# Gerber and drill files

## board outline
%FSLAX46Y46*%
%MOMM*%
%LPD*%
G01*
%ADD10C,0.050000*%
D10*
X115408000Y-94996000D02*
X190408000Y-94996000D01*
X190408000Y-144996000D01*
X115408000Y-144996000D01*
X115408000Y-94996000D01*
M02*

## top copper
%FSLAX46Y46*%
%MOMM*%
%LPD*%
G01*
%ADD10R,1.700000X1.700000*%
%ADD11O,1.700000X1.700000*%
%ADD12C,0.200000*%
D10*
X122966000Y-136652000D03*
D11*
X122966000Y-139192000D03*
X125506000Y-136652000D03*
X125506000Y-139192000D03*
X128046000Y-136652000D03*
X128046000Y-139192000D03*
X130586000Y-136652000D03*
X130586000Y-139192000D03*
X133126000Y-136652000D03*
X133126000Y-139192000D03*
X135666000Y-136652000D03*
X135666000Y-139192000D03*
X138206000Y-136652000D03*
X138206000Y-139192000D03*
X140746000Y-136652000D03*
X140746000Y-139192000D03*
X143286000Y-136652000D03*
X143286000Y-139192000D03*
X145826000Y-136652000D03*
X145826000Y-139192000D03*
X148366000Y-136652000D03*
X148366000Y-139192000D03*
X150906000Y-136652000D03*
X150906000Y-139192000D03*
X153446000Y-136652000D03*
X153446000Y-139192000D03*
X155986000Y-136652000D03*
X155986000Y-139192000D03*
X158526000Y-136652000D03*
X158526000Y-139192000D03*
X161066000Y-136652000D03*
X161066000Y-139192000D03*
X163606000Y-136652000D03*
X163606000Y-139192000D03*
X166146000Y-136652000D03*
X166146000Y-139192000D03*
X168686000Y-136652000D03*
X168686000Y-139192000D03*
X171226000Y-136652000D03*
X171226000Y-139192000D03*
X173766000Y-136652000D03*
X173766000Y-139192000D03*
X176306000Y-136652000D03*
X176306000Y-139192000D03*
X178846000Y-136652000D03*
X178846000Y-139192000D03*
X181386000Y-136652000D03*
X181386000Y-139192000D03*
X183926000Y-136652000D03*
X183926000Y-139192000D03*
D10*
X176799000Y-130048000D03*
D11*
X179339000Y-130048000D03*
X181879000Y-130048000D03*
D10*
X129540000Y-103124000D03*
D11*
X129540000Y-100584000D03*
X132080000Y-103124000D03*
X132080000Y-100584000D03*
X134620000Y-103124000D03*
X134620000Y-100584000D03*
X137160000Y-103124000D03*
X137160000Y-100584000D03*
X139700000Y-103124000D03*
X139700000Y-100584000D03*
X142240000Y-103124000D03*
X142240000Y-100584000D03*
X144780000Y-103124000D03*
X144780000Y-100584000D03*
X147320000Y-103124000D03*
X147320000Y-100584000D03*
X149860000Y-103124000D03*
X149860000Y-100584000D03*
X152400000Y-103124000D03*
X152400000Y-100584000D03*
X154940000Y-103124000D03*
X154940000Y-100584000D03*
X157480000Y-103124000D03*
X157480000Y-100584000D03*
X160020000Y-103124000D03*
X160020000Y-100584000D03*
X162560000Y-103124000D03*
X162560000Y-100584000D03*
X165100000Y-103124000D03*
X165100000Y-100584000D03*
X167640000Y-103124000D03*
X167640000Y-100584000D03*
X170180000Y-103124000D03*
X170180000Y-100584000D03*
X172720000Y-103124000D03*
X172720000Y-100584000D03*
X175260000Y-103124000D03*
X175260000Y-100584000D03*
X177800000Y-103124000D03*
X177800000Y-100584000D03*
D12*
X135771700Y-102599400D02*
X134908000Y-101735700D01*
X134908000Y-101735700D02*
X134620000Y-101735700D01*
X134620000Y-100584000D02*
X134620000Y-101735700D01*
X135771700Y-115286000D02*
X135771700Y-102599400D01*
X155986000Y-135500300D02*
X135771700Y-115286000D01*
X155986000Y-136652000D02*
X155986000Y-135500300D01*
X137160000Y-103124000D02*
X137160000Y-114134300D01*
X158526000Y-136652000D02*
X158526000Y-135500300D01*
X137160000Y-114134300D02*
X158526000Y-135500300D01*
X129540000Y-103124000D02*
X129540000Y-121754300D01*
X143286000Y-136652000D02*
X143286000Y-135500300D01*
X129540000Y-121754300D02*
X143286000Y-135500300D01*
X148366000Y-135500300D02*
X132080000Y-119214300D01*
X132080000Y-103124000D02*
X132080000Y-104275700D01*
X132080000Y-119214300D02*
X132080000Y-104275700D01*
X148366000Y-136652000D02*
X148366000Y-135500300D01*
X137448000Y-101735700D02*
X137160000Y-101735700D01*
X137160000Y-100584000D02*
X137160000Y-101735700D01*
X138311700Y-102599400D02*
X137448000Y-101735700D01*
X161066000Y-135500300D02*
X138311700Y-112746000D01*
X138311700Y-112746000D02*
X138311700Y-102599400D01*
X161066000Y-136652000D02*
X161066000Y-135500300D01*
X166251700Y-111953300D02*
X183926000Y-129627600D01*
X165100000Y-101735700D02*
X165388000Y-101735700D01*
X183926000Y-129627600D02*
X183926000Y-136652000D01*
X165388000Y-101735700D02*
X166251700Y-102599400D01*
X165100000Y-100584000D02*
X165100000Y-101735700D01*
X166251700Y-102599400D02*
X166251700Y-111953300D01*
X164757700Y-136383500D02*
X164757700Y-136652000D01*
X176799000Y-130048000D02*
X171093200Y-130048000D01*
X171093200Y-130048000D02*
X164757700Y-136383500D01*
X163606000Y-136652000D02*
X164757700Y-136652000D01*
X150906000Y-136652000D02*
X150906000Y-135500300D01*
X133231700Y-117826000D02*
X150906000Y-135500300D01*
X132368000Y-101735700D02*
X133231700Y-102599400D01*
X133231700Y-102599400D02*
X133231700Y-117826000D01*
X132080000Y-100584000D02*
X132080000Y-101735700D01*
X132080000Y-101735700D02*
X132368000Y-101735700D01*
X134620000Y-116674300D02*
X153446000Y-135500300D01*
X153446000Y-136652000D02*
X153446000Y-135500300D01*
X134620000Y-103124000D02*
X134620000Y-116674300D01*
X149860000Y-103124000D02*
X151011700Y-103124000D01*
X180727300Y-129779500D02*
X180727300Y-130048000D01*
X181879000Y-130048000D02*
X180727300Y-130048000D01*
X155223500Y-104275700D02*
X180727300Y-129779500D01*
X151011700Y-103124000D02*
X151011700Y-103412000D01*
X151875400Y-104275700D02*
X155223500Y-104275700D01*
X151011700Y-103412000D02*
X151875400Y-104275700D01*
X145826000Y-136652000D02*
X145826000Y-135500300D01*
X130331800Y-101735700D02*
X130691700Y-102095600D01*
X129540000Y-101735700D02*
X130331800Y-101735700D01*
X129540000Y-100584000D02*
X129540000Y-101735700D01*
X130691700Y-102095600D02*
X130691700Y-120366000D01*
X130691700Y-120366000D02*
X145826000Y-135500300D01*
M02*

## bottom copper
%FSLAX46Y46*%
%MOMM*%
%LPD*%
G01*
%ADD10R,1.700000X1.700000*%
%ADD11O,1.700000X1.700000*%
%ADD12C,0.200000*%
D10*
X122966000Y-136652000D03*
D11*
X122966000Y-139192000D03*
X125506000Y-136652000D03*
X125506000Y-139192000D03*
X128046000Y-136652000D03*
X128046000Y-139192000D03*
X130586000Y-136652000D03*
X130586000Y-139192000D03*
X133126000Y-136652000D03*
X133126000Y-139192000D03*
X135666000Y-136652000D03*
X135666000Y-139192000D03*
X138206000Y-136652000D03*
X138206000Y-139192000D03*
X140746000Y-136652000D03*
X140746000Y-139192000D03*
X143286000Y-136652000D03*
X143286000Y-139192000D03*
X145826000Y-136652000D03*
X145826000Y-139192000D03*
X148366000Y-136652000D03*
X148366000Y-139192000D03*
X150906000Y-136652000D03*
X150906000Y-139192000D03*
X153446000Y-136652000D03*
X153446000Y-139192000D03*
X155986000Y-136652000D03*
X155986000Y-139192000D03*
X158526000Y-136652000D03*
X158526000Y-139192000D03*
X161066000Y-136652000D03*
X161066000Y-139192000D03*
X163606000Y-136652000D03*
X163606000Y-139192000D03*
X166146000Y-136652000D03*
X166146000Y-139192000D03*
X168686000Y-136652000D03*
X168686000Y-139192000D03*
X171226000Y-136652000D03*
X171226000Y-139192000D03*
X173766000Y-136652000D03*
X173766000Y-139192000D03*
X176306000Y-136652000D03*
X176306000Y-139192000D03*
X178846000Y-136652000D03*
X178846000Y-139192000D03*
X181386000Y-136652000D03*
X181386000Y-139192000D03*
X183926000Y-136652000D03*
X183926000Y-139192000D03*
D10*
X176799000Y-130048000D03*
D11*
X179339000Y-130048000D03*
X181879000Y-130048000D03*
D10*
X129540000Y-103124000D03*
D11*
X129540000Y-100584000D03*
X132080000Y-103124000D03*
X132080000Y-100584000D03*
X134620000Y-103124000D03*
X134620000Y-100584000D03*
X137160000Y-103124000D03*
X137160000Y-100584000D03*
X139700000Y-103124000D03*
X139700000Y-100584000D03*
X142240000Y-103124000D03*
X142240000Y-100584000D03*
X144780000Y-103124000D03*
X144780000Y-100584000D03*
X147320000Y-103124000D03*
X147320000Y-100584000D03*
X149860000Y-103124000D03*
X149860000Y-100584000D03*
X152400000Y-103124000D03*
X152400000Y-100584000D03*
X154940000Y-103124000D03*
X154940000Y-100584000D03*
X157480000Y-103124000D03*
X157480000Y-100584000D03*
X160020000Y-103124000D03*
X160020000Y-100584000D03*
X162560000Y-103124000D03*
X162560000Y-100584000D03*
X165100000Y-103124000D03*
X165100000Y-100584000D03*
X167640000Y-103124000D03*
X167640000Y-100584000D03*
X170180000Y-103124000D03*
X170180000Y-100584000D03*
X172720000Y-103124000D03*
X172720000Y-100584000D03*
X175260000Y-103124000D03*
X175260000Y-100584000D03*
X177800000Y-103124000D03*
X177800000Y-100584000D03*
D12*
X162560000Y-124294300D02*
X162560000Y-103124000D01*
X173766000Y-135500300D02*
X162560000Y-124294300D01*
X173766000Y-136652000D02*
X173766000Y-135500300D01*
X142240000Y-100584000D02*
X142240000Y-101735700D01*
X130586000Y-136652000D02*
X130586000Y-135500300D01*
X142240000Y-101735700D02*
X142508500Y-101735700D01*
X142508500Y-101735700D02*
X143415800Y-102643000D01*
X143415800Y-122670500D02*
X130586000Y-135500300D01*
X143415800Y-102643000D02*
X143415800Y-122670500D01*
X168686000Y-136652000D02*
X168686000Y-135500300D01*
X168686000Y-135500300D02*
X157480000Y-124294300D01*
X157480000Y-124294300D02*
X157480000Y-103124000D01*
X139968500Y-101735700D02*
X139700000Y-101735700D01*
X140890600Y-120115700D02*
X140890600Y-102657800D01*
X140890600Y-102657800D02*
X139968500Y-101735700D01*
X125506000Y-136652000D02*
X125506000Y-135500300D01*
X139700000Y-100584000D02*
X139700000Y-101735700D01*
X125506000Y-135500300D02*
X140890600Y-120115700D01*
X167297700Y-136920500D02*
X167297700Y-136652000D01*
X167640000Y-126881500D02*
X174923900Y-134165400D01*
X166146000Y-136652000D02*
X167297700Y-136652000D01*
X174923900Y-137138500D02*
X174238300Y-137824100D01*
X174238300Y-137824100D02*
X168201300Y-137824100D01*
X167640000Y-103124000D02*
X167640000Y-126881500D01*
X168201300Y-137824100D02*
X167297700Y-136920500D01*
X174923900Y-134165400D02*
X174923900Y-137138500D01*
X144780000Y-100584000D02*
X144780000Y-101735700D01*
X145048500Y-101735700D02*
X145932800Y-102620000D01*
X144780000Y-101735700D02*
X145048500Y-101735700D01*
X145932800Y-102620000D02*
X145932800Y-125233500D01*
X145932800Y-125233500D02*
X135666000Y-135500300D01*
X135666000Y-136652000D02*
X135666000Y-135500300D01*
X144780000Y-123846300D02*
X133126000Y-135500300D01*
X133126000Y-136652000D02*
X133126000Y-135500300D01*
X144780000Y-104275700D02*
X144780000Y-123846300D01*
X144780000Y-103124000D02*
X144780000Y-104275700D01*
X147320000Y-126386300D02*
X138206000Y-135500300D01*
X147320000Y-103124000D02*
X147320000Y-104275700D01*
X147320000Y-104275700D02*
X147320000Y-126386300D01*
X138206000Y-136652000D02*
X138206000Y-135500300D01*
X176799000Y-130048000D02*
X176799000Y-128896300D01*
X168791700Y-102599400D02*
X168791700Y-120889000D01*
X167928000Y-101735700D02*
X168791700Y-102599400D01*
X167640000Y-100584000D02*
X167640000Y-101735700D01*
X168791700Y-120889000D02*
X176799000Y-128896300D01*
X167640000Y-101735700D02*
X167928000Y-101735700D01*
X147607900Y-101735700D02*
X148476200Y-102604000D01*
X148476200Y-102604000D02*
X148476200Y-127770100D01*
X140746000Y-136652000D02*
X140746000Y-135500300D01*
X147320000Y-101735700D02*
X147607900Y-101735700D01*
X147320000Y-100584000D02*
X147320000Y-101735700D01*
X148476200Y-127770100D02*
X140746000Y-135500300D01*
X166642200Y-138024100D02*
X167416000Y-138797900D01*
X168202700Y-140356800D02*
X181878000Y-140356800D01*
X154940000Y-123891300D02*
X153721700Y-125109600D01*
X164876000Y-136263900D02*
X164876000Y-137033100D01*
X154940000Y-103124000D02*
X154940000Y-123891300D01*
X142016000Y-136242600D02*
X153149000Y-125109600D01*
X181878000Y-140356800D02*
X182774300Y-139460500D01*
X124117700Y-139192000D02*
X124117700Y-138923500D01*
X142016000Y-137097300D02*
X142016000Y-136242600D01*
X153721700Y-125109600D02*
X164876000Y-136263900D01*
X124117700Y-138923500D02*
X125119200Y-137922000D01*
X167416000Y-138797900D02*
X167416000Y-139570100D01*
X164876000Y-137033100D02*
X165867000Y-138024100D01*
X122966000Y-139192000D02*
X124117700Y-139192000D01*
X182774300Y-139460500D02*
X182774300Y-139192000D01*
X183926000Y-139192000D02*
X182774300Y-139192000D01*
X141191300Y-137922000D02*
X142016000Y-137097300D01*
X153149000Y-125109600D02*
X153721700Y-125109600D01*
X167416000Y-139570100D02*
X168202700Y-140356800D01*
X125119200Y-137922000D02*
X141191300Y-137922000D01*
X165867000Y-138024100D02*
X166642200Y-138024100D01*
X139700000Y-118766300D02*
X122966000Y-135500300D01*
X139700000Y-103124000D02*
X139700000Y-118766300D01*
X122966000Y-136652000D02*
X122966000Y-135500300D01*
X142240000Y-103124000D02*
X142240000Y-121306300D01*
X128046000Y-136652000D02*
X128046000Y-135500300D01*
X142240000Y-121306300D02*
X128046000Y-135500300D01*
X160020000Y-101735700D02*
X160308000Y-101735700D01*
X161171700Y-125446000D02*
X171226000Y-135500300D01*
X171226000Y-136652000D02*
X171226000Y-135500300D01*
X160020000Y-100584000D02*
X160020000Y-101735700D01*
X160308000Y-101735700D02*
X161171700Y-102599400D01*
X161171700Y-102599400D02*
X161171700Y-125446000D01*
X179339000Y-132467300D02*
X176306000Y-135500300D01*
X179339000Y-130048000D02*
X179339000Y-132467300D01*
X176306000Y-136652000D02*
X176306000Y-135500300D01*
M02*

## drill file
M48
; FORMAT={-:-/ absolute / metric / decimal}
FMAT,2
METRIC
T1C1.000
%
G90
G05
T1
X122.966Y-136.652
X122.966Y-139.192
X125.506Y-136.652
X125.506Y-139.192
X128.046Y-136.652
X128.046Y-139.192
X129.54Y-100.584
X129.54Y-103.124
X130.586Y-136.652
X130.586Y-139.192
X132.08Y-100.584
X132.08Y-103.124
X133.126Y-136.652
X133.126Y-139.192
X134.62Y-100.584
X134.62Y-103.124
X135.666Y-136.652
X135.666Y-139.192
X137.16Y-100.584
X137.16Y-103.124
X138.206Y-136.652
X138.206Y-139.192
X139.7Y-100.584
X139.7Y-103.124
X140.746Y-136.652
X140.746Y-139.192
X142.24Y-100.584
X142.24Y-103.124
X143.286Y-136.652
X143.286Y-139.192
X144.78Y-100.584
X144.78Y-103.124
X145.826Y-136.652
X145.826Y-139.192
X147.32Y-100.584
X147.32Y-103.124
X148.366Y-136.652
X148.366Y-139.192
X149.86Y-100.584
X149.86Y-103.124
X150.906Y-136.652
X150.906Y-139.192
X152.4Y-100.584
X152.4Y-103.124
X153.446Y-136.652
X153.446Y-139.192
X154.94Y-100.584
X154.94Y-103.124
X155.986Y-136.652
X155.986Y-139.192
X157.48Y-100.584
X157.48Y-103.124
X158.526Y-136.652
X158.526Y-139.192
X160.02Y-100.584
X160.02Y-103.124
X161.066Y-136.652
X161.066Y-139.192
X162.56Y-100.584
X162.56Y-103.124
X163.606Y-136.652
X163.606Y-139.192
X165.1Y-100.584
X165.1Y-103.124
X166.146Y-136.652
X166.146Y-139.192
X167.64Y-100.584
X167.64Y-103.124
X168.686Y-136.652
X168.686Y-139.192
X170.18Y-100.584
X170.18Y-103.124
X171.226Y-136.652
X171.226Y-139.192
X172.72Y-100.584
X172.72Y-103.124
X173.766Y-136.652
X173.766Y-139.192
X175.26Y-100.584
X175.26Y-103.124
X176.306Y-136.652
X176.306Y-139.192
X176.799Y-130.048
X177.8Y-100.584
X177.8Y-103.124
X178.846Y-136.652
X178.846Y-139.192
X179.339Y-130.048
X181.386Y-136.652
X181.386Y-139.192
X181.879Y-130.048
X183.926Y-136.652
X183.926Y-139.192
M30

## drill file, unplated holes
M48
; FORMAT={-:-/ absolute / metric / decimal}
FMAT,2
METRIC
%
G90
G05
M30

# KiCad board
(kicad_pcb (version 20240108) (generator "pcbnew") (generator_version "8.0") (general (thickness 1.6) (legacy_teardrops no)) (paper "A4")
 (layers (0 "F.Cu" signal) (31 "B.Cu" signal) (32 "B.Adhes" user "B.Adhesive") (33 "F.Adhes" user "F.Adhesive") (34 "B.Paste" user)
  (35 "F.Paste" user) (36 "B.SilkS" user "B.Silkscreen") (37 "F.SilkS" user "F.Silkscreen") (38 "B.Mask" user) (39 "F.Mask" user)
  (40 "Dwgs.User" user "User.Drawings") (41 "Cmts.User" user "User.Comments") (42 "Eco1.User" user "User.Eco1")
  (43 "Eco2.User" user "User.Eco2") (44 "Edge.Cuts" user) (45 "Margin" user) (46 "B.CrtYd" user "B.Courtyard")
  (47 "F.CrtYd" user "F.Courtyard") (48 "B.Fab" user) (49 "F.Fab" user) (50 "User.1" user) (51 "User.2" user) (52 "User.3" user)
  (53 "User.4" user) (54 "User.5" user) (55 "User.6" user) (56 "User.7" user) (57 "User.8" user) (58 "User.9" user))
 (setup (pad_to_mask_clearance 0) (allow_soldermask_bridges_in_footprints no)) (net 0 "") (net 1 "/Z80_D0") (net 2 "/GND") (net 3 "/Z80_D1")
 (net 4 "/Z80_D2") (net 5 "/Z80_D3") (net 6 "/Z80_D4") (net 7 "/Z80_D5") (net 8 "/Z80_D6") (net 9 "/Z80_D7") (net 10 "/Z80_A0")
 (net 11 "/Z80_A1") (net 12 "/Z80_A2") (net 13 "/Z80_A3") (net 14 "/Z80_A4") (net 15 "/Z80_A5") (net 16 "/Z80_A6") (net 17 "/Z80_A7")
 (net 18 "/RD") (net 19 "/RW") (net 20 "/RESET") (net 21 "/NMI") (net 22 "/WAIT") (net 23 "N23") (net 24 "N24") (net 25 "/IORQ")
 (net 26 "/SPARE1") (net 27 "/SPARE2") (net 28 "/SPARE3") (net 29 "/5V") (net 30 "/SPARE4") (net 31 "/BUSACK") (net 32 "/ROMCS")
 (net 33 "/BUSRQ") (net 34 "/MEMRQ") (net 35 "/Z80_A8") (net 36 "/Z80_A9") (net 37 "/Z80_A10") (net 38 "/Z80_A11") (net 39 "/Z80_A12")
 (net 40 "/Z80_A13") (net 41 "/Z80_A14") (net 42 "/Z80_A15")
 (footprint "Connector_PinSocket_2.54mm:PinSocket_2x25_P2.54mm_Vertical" (layer "F.Cu") (at 122.966 136.652 90)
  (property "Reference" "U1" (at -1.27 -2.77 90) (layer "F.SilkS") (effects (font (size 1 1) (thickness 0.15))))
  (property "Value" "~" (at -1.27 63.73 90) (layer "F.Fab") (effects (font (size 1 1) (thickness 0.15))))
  (pad "1" thru_hole rect (at 0 0 90) (size 1.7 1.7) (drill 1) (layers "*.Cu" "*.Mask") (remove_unused_layers no) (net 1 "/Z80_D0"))
  (pad "2" thru_hole oval (at -2.54 0 90) (size 1.7 1.7) (drill 1) (layers "*.Cu" "*.Mask") (remove_unused_layers no) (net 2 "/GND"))
  (pad "3" thru_hole oval (at 0 2.54 90) (size 1.7 1.7) (drill 1) (layers "*.Cu" "*.Mask") (remove_unused_layers no) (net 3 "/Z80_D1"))
  (pad "4" thru_hole oval (at -2.54 2.54 90) (size 1.7 1.7) (drill 1) (layers "*.Cu" "*.Mask") (remove_unused_layers no))
  (pad "5" thru_hole oval (at 0 5.08 90) (size 1.7 1.7) (drill 1) (layers "*.Cu" "*.Mask") (remove_unused_layers no) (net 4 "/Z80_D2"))
  (pad "6" thru_hole oval (at -2.54 5.08 90) (size 1.7 1.7) (drill 1) (layers "*.Cu" "*.Mask") (remove_unused_layers no))
  (pad "7" thru_hole oval (at 0 7.62 90) (size 1.7 1.7) (drill 1) (layers "*.Cu" "*.Mask") (remove_unused_layers no) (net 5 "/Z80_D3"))
  (pad "8" thru_hole oval (at -2.54 7.62 90) (size 1.7 1.7) (drill 1) (layers "*.Cu" "*.Mask") (remove_unused_layers no))
  (pad "9" thru_hole oval (at 0 10.16 90) (size 1.7 1.7) (drill 1) (layers "*.Cu" "*.Mask") (remove_unused_layers no) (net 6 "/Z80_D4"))
  (pad "10" thru_hole oval (at -2.54 10.16 90) (size 1.7 1.7) (drill 1) (layers "*.Cu" "*.Mask") (remove_unused_layers no))
  (pad "11" thru_hole oval (at 0 12.7 90) (size 1.7 1.7) (drill 1) (layers "*.Cu" "*.Mask") (remove_unused_layers no) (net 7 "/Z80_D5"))
  (pad "12" thru_hole oval (at -2.54 12.7 90) (size 1.7 1.7) (drill 1) (layers "*.Cu" "*.Mask") (remove_unused_layers no))
  (pad "13" thru_hole oval (at 0 15.24 90) (size 1.7 1.7) (drill 1) (layers "*.Cu" "*.Mask") (remove_unused_layers no) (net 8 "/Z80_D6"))
  (pad "14" thru_hole oval (at -2.54 15.24 90) (size 1.7 1.7) (drill 1) (layers "*.Cu" "*.Mask") (remove_unused_layers no))
  (pad "15" thru_hole oval (at 0 17.78 90) (size 1.7 1.7) (drill 1) (layers "*.Cu" "*.Mask") (remove_unused_layers no) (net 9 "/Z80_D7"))
  (pad "16" thru_hole oval (at -2.54 17.78 90) (size 1.7 1.7) (drill 1) (layers "*.Cu" "*.Mask") (remove_unused_layers no))
  (pad "17" thru_hole oval (at 0 20.32 90) (size 1.7 1.7) (drill 1) (layers "*.Cu" "*.Mask") (remove_unused_layers no) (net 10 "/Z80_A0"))
  (pad "18" thru_hole oval (at -2.54 20.32 90) (size 1.7 1.7) (drill 1) (layers "*.Cu" "*.Mask") (remove_unused_layers no))
  (pad "19" thru_hole oval (at 0 22.86 90) (size 1.7 1.7) (drill 1) (layers "*.Cu" "*.Mask") (remove_unused_layers no) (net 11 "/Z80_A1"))
  (pad "20" thru_hole oval (at -2.54 22.86 90) (size 1.7 1.7) (drill 1) (layers "*.Cu" "*.Mask") (remove_unused_layers no))
  (pad "21" thru_hole oval (at 0 25.4 90) (size 1.7 1.7) (drill 1) (layers "*.Cu" "*.Mask") (remove_unused_layers no) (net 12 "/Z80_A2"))
  (pad "22" thru_hole oval (at -2.54 25.4 90) (size 1.7 1.7) (drill 1) (layers "*.Cu" "*.Mask") (remove_unused_layers no))
  (pad "23" thru_hole oval (at 0 27.94 90) (size 1.7 1.7) (drill 1) (layers "*.Cu" "*.Mask") (remove_unused_layers no) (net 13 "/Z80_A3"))
  (pad "24" thru_hole oval (at -2.54 27.94 90) (size 1.7 1.7) (drill 1) (layers "*.Cu" "*.Mask") (remove_unused_layers no))
  (pad "25" thru_hole oval (at 0 30.48 90) (size 1.7 1.7) (drill 1) (layers "*.Cu" "*.Mask") (remove_unused_layers no) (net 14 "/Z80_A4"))
  (pad "26" thru_hole oval (at -2.54 30.48 90) (size 1.7 1.7) (drill 1) (layers "*.Cu" "*.Mask") (remove_unused_layers no))
  (pad "27" thru_hole oval (at 0 33.02 90) (size 1.7 1.7) (drill 1) (layers "*.Cu" "*.Mask") (remove_unused_layers no) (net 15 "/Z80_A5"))
  (pad "28" thru_hole oval (at -2.54 33.02 90) (size 1.7 1.7) (drill 1) (layers "*.Cu" "*.Mask") (remove_unused_layers no))
  (pad "29" thru_hole oval (at 0 35.56 90) (size 1.7 1.7) (drill 1) (layers "*.Cu" "*.Mask") (remove_unused_layers no) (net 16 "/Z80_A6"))
  (pad "30" thru_hole oval (at -2.54 35.56 90) (size 1.7 1.7) (drill 1) (layers "*.Cu" "*.Mask") (remove_unused_layers no))
  (pad "31" thru_hole oval (at 0 38.1 90) (size 1.7 1.7) (drill 1) (layers "*.Cu" "*.Mask") (remove_unused_layers no) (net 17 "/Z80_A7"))
  (pad "32" thru_hole oval (at -2.54 38.1 90) (size 1.7 1.7) (drill 1) (layers "*.Cu" "*.Mask") (remove_unused_layers no))
  (pad "33" thru_hole oval (at 0 40.64 90) (size 1.7 1.7) (drill 1) (layers "*.Cu" "*.Mask") (remove_unused_layers no) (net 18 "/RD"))
  (pad "34" thru_hole oval (at -2.54 40.64 90) (size 1.7 1.7) (drill 1) (layers "*.Cu" "*.Mask") (remove_unused_layers no))
  (pad "35" thru_hole oval (at 0 43.18 90) (size 1.7 1.7) (drill 1) (layers "*.Cu" "*.Mask") (remove_unused_layers no) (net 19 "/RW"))
  (pad "36" thru_hole oval (at -2.54 43.18 90) (size 1.7 1.7) (drill 1) (layers "*.Cu" "*.Mask") (remove_unused_layers no))
  (pad "37" thru_hole oval (at 0 45.72 90) (size 1.7 1.7) (drill 1) (layers "*.Cu" "*.Mask") (remove_unused_layers no) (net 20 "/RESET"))
  (pad "38" thru_hole oval (at -2.54 45.72 90) (size 1.7 1.7) (drill 1) (layers "*.Cu" "*.Mask") (remove_unused_layers no))
  (pad "39" thru_hole oval (at 0 48.26 90) (size 1.7 1.7) (drill 1) (layers "*.Cu" "*.Mask") (remove_unused_layers no) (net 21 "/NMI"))
  (pad "40" thru_hole oval (at -2.54 48.26 90) (size 1.7 1.7) (drill 1) (layers "*.Cu" "*.Mask") (remove_unused_layers no))
  (pad "41" thru_hole oval (at 0 50.8 90) (size 1.7 1.7) (drill 1) (layers "*.Cu" "*.Mask") (remove_unused_layers no) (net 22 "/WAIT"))
  (pad "42" thru_hole oval (at -2.54 50.8 90) (size 1.7 1.7) (drill 1) (layers "*.Cu" "*.Mask") (remove_unused_layers no))
  (pad "43" thru_hole oval (at 0 53.34 90) (size 1.7 1.7) (drill 1) (layers "*.Cu" "*.Mask") (remove_unused_layers no) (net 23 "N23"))
  (pad "44" thru_hole oval (at -2.54 53.34 90) (size 1.7 1.7) (drill 1) (layers "*.Cu" "*.Mask") (remove_unused_layers no))
  (pad "45" thru_hole oval (at 0 55.88 90) (size 1.7 1.7) (drill 1) (layers "*.Cu" "*.Mask") (remove_unused_layers no))
  (pad "46" thru_hole oval (at -2.54 55.88 90) (size 1.7 1.7) (drill 1) (layers "*.Cu" "*.Mask") (remove_unused_layers no))
  (pad "47" thru_hole oval (at 0 58.42 90) (size 1.7 1.7) (drill 1) (layers "*.Cu" "*.Mask") (remove_unused_layers no) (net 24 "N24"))
  (pad "48" thru_hole oval (at -2.54 58.42 90) (size 1.7 1.7) (drill 1) (layers "*.Cu" "*.Mask") (remove_unused_layers no))
  (pad "49" thru_hole oval (at 0 60.96 90) (size 1.7 1.7) (drill 1) (layers "*.Cu" "*.Mask") (remove_unused_layers no) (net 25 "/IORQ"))
  (pad "50" thru_hole oval (at -2.54 60.96 90) (size 1.7 1.7) (drill 1) (layers "*.Cu" "*.Mask") (remove_unused_layers no) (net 2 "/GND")))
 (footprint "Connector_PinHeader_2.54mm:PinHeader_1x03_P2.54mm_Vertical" (layer "F.Cu") (at 176.799 130.048 90)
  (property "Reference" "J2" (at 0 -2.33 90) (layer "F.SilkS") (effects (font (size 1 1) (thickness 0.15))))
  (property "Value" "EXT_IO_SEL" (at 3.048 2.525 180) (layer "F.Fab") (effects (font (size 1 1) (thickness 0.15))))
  (pad "1" thru_hole rect (at 0 0 90) (size 1.7 1.7) (drill 1) (layers "*.Cu" "*.Mask") (remove_unused_layers no) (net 18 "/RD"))
  (pad "2" thru_hole oval (at 0 2.54 90) (size 1.7 1.7) (drill 1) (layers "*.Cu" "*.Mask") (remove_unused_layers no) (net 23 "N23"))
  (pad "3" thru_hole oval (at 0 5.08 90) (size 1.7 1.7) (drill 1) (layers "*.Cu" "*.Mask") (remove_unused_layers no) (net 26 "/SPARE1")))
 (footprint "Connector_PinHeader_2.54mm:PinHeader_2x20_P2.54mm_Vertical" (layer "F.Cu") (at 129.54 103.124 90)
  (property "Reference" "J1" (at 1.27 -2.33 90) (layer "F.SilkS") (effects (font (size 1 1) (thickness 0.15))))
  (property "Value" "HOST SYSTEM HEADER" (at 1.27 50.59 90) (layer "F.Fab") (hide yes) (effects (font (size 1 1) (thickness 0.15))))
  (pad "1" thru_hole rect (at 0 0 90) (size 1.7 1.7) (drill 1) (layers "*.Cu" "*.Mask") (remove_unused_layers no) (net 10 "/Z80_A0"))
  (pad "2" thru_hole oval (at 2.54 0 90) (size 1.7 1.7) (drill 1) (layers "*.Cu" "*.Mask") (remove_unused_layers no) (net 11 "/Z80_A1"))
  (pad "3" thru_hole oval (at 0 2.54 90) (size 1.7 1.7) (drill 1) (layers "*.Cu" "*.Mask") (remove_unused_layers no) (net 12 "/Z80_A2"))
  (pad "4" thru_hole oval (at 2.54 2.54 90) (size 1.7 1.7) (drill 1) (layers "*.Cu" "*.Mask") (remove_unused_layers no) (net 13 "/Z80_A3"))
  (pad "5" thru_hole oval (at 0 5.08 90) (size 1.7 1.7) (drill 1) (layers "*.Cu" "*.Mask") (remove_unused_layers no) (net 14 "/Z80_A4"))
  (pad "6" thru_hole oval (at 2.54 5.08 90) (size 1.7 1.7) (drill 1) (layers "*.Cu" "*.Mask") (remove_unused_layers no) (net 15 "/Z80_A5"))
  (pad "7" thru_hole oval (at 0 7.62 90) (size 1.7 1.7) (drill 1) (layers "*.Cu" "*.Mask") (remove_unused_layers no) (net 16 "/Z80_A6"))
  (pad "8" thru_hole oval (at 2.54 7.62 90) (size 1.7 1.7) (drill 1) (layers "*.Cu" "*.Mask") (remove_unused_layers no) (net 17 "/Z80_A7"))
  (pad "9" thru_hole oval (at 0 10.16 90) (size 1.7 1.7) (drill 1) (layers "*.Cu" "*.Mask") (remove_unused_layers no) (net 1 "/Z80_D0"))
  (pad "10" thru_hole oval (at 2.54 10.16 90) (size 1.7 1.7) (drill 1) (layers "*.Cu" "*.Mask") (remove_unused_layers no) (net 3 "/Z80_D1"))
  (pad "11" thru_hole oval (at 0 12.7 90) (size 1.7 1.7) (drill 1) (layers "*.Cu" "*.Mask") (remove_unused_layers no) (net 4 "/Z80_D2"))
  (pad "12" thru_hole oval (at 2.54 12.7 90) (size 1.7 1.7) (drill 1) (layers "*.Cu" "*.Mask") (remove_unused_layers no) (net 5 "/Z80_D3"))
  (pad "13" thru_hole oval (at 0 15.24 90) (size 1.7 1.7) (drill 1) (layers "*.Cu" "*.Mask") (remove_unused_layers no) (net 6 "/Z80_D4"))
  (pad "14" thru_hole oval (at 2.54 15.24 90) (size 1.7 1.7) (drill 1) (layers "*.Cu" "*.Mask") (remove_unused_layers no) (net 7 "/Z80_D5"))
  (pad "15" thru_hole oval (at 0 17.78 90) (size 1.7 1.7) (drill 1) (layers "*.Cu" "*.Mask") (remove_unused_layers no) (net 8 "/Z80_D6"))
  (pad "16" thru_hole oval (at 2.54 17.78 90) (size 1.7 1.7) (drill 1) (layers "*.Cu" "*.Mask") (remove_unused_layers no) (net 9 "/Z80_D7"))
  (pad "17" thru_hole oval (at 0 20.32 90) (size 1.7 1.7) (drill 1) (layers "*.Cu" "*.Mask") (remove_unused_layers no) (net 26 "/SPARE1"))
  (pad "18" thru_hole oval (at 2.54 20.32 90) (size 1.7 1.7) (drill 1) (layers "*.Cu" "*.Mask") (remove_unused_layers no) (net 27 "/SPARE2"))
  (pad "19" thru_hole oval (at 0 22.86 90) (size 1.7 1.7) (drill 1) (layers "*.Cu" "*.Mask") (remove_unused_layers no) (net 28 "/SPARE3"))
  (pad "20" thru_hole oval (at 2.54 22.86 90) (size 1.7 1.7) (drill 1) (layers "*.Cu" "*.Mask") (remove_unused_layers no) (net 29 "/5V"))
  (pad "21" thru_hole oval (at 0 25.4 90) (size 1.7 1.7) (drill 1) (layers "*.Cu" "*.Mask") (remove_unused_layers no) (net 2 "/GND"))
  (pad "22" thru_hole oval (at 2.54 25.4 90) (size 1.7 1.7) (drill 1) (layers "*.Cu" "*.Mask") (remove_unused_layers no) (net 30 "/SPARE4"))
  (pad "23" thru_hole oval (at 0 27.94 90) (size 1.7 1.7) (drill 1) (layers "*.Cu" "*.Mask") (remove_unused_layers no) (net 20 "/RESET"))
  (pad "24" thru_hole oval (at 2.54 27.94 90) (size 1.7 1.7) (drill 1) (layers "*.Cu" "*.Mask") (remove_unused_layers no) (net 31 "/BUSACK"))
  (pad "25" thru_hole oval (at 0 30.48 90) (size 1.7 1.7) (drill 1) (layers "*.Cu" "*.Mask") (remove_unused_layers no) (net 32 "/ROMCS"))
  (pad "26" thru_hole oval (at 2.54 30.48 90) (size 1.7 1.7) (drill 1) (layers "*.Cu" "*.Mask") (remove_unused_layers no) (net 21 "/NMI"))
  (pad "27" thru_hole oval (at 0 33.02 90) (size 1.7 1.7) (drill 1) (layers "*.Cu" "*.Mask") (remove_unused_layers no) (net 22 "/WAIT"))
  (pad "28" thru_hole oval (at 2.54 33.02 90) (size 1.7 1.7) (drill 1) (layers "*.Cu" "*.Mask") (remove_unused_layers no) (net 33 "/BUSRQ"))
  (pad "29" thru_hole oval (at 0 35.56 90) (size 1.7 1.7) (drill 1) (layers "*.Cu" "*.Mask") (remove_unused_layers no) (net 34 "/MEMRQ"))
  (pad "30" thru_hole oval (at 2.54 35.56 90) (size 1.7 1.7) (drill 1) (layers "*.Cu" "*.Mask") (remove_unused_layers no) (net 25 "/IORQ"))
  (pad "31" thru_hole oval (at 0 38.1 90) (size 1.7 1.7) (drill 1) (layers "*.Cu" "*.Mask") (remove_unused_layers no) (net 19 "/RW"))
  (pad "32" thru_hole oval (at 2.54 38.1 90) (size 1.7 1.7) (drill 1) (layers "*.Cu" "*.Mask") (remove_unused_layers no) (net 18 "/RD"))
  (pad "33" thru_hole oval (at 0 40.64 90) (size 1.7 1.7) (drill 1) (layers "*.Cu" "*.Mask") (remove_unused_layers no) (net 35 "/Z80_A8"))
  (pad "34" thru_hole oval (at 2.54 40.64 90) (size 1.7 1.7) (drill 1) (layers "*.Cu" "*.Mask") (remove_unused_layers no) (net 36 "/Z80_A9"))
  (pad "35" thru_hole oval (at 0 43.18 90) (size 1.7 1.7) (drill 1) (layers "*.Cu" "*.Mask") (remove_unused_layers no) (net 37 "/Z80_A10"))
  (pad "36" thru_hole oval (at 2.54 43.18 90) (size 1.7 1.7) (drill 1) (layers "*.Cu" "*.Mask") (remove_unused_layers no)
   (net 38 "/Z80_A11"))
  (pad "37" thru_hole oval (at 0 45.72 90) (size 1.7 1.7) (drill 1) (layers "*.Cu" "*.Mask") (remove_unused_layers no) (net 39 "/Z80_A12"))
  (pad "38" thru_hole oval (at 2.54 45.72 90) (size 1.7 1.7) (drill 1) (layers "*.Cu" "*.Mask") (remove_unused_layers no)
   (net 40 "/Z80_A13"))
  (pad "39" thru_hole oval (at 0 48.26 90) (size 1.7 1.7) (drill 1) (layers "*.Cu" "*.Mask") (remove_unused_layers no) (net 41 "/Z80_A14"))
  (pad "40" thru_hole oval (at 2.54 48.26 90) (size 1.7 1.7) (drill 1) (layers "*.Cu" "*.Mask") (remove_unused_layers no)
   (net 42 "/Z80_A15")))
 (gr_rect (start 115.408 94.996) (end 190.408 144.996) (stroke (width 0.05) (type default)) (fill none) (layer "Edge.Cuts"))
 (segment (start 135.7717 102.5994) (end 134.908 101.7357) (width 0.2) (layer "F.Cu") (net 15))
 (segment (start 134.908 101.7357) (end 134.62 101.7357) (width 0.2) (layer "F.Cu") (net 15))
 (segment (start 134.62 100.584) (end 134.62 101.7357) (width 0.2) (layer "F.Cu") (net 15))
 (segment (start 135.7717 115.286) (end 135.7717 102.5994) (width 0.2) (layer "F.Cu") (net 15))
 (segment (start 155.986 135.5003) (end 135.7717 115.286) (width 0.2) (layer "F.Cu") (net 15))
 (segment (start 155.986 136.652) (end 155.986 135.5003) (width 0.2) (layer "F.Cu") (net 15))
 (segment (start 137.16 103.124) (end 137.16 114.1343) (width 0.2) (layer "F.Cu") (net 16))
 (segment (start 158.526 136.652) (end 158.526 135.5003) (width 0.2) (layer "F.Cu") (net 16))
 (segment (start 137.16 114.1343) (end 158.526 135.5003) (width 0.2) (layer "F.Cu") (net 16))
 (segment (start 162.56 124.2943) (end 162.56 103.124) (width 0.2) (layer "B.Cu") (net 22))
 (segment (start 173.766 135.5003) (end 162.56 124.2943) (width 0.2) (layer "B.Cu") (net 22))
 (segment (start 173.766 136.652) (end 173.766 135.5003) (width 0.2) (layer "B.Cu") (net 22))
 (segment (start 142.24 100.584) (end 142.24 101.7357) (width 0.2) (layer "B.Cu") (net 5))
 (segment (start 130.586 136.652) (end 130.586 135.5003) (width 0.2) (layer "B.Cu") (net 5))
 (segment (start 142.24 101.7357) (end 142.5085 101.7357) (width 0.2) (layer "B.Cu") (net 5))
 (segment (start 142.5085 101.7357) (end 143.4158 102.643) (width 0.2) (layer "B.Cu") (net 5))
 (segment (start 143.4158 122.6705) (end 130.586 135.5003) (width 0.2) (layer "B.Cu") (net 5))
 (segment (start 143.4158 102.643) (end 143.4158 122.6705) (width 0.2) (layer "B.Cu") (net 5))
 (segment (start 168.686 136.652) (end 168.686 135.5003) (width 0.2) (layer "B.Cu") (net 20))
 (segment (start 168.686 135.5003) (end 157.48 124.2943) (width 0.2) (layer "B.Cu") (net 20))
 (segment (start 157.48 124.2943) (end 157.48 103.124) (width 0.2) (layer "B.Cu") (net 20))
 (segment (start 139.9685 101.7357) (end 139.7 101.7357) (width 0.2) (layer "B.Cu") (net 3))
 (segment (start 140.8906 120.1157) (end 140.8906 102.6578) (width 0.2) (layer "B.Cu") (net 3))
 (segment (start 140.8906 102.6578) (end 139.9685 101.7357) (width 0.2) (layer "B.Cu") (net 3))
 (segment (start 125.506 136.652) (end 125.506 135.5003) (width 0.2) (layer "B.Cu") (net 3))
 (segment (start 139.7 100.584) (end 139.7 101.7357) (width 0.2) (layer "B.Cu") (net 3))
 (segment (start 125.506 135.5003) (end 140.8906 120.1157) (width 0.2) (layer "B.Cu") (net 3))
 (segment (start 167.2977 136.9205) (end 167.2977 136.652) (width 0.2) (layer "B.Cu") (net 19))
 (segment (start 167.64 126.8815) (end 174.9239 134.1654) (width 0.2) (layer "B.Cu") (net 19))
 (segment (start 166.146 136.652) (end 167.2977 136.652) (width 0.2) (layer "B.Cu") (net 19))
 (segment (start 174.9239 137.1385) (end 174.2383 137.8241) (width 0.2) (layer "B.Cu") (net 19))
 (segment (start 174.2383 137.8241) (end 168.2013 137.8241) (width 0.2) (layer "B.Cu") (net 19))
 (segment (start 167.64 103.124) (end 167.64 126.8815) (width 0.2) (layer "B.Cu") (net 19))
 (segment (start 168.2013 137.8241) (end 167.2977 136.9205) (width 0.2) (layer "B.Cu") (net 19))
 (segment (start 174.9239 134.1654) (end 174.9239 137.1385) (width 0.2) (layer "B.Cu") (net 19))
 (segment (start 144.78 100.584) (end 144.78 101.7357) (width 0.2) (layer "B.Cu") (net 7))
 (segment (start 145.0485 101.7357) (end 145.9328 102.62) (width 0.2) (layer "B.Cu") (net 7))
 (segment (start 144.78 101.7357) (end 145.0485 101.7357) (width 0.2) (layer "B.Cu") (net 7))
 (segment (start 145.9328 102.62) (end 145.9328 125.2335) (width 0.2) (layer "B.Cu") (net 7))
 (segment (start 145.9328 125.2335) (end 135.666 135.5003) (width 0.2) (layer "B.Cu") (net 7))
 (segment (start 135.666 136.652) (end 135.666 135.5003) (width 0.2) (layer "B.Cu") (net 7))
 (segment (start 144.78 123.8463) (end 133.126 135.5003) (width 0.2) (layer "B.Cu") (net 6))
 (segment (start 133.126 136.652) (end 133.126 135.5003) (width 0.2) (layer "B.Cu") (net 6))
 (segment (start 144.78 104.2757) (end 144.78 123.8463) (width 0.2) (layer "B.Cu") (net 6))
 (segment (start 144.78 103.124) (end 144.78 104.2757) (width 0.2) (layer "B.Cu") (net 6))
 (segment (start 147.32 126.3863) (end 138.206 135.5003) (width 0.2) (layer "B.Cu") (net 8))
 (segment (start 147.32 103.124) (end 147.32 104.2757) (width 0.2) (layer "B.Cu") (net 8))
 (segment (start 147.32 104.2757) (end 147.32 126.3863) (width 0.2) (layer "B.Cu") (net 8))
 (segment (start 138.206 136.652) (end 138.206 135.5003) (width 0.2) (layer "B.Cu") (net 8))
 (segment (start 129.54 103.124) (end 129.54 121.7543) (width 0.2) (layer "F.Cu") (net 10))
 (segment (start 143.286 136.652) (end 143.286 135.5003) (width 0.2) (layer "F.Cu") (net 10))
 (segment (start 129.54 121.7543) (end 143.286 135.5003) (width 0.2) (layer "F.Cu") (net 10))
 (segment (start 148.366 135.5003) (end 132.08 119.2143) (width 0.2) (layer "F.Cu") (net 12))
 (segment (start 132.08 103.124) (end 132.08 104.2757) (width 0.2) (layer "F.Cu") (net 12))
 (segment (start 132.08 119.2143) (end 132.08 104.2757) (width 0.2) (layer "F.Cu") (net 12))
 (segment (start 148.366 136.652) (end 148.366 135.5003) (width 0.2) (layer "F.Cu") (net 12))
 (segment (start 137.448 101.7357) (end 137.16 101.7357) (width 0.2) (layer "F.Cu") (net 17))
 (segment (start 137.16 100.584) (end 137.16 101.7357) (width 0.2) (layer "F.Cu") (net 17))
 (segment (start 138.3117 102.5994) (end 137.448 101.7357) (width 0.2) (layer "F.Cu") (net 17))
 (segment (start 161.066 135.5003) (end 138.3117 112.746) (width 0.2) (layer "F.Cu") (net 17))
 (segment (start 138.3117 112.746) (end 138.3117 102.5994) (width 0.2) (layer "F.Cu") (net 17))
 (segment (start 161.066 136.652) (end 161.066 135.5003) (width 0.2) (layer "F.Cu") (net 17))
 (segment (start 166.2517 111.9533) (end 183.926 129.6276) (width 0.2) (layer "F.Cu") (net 25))
 (segment (start 165.1 101.7357) (end 165.388 101.7357) (width 0.2) (layer "F.Cu") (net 25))
 (segment (start 183.926 129.6276) (end 183.926 136.652) (width 0.2) (layer "F.Cu") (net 25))
 (segment (start 165.388 101.7357) (end 166.2517 102.5994) (width 0.2) (layer "F.Cu") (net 25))
 (segment (start 165.1 100.584) (end 165.1 101.7357) (width 0.2) (layer "F.Cu") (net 25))
 (segment (start 166.2517 102.5994) (end 166.2517 111.9533) (width 0.2) (layer "F.Cu") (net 25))
 (segment (start 164.7577 136.3835) (end 164.7577 136.652) (width 0.2) (layer "F.Cu") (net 18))
 (segment (start 176.799 130.048) (end 171.0932 130.048) (width 0.2) (layer "F.Cu") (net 18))
 (segment (start 171.0932 130.048) (end 164.7577 136.3835) (width 0.2) (layer "F.Cu") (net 18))
 (segment (start 163.606 136.652) (end 164.7577 136.652) (width 0.2) (layer "F.Cu") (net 18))
 (segment (start 176.799 130.048) (end 176.799 128.8963) (width 0.2) (layer "B.Cu") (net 18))
 (segment (start 168.7917 102.5994) (end 168.7917 120.889) (width 0.2) (layer "B.Cu") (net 18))
 (segment (start 167.928 101.7357) (end 168.7917 102.5994) (width 0.2) (layer "B.Cu") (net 18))
 (segment (start 167.64 100.584) (end 167.64 101.7357) (width 0.2) (layer "B.Cu") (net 18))
 (segment (start 168.7917 120.889) (end 176.799 128.8963) (width 0.2) (layer "B.Cu") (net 18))
 (segment (start 167.64 101.7357) (end 167.928 101.7357) (width 0.2) (layer "B.Cu") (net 18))
 (segment (start 147.6079 101.7357) (end 148.4762 102.604) (width 0.2) (layer "B.Cu") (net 9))
 (segment (start 148.4762 102.604) (end 148.4762 127.7701) (width 0.2) (layer "B.Cu") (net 9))
 (segment (start 140.746 136.652) (end 140.746 135.5003) (width 0.2) (layer "B.Cu") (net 9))
 (segment (start 147.32 101.7357) (end 147.6079 101.7357) (width 0.2) (layer "B.Cu") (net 9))
 (segment (start 147.32 100.584) (end 147.32 101.7357) (width 0.2) (layer "B.Cu") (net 9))
 (segment (start 148.4762 127.7701) (end 140.746 135.5003) (width 0.2) (layer "B.Cu") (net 9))
 (segment (start 150.906 136.652) (end 150.906 135.5003) (width 0.2) (layer "F.Cu") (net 13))
 (segment (start 133.2317 117.826) (end 150.906 135.5003) (width 0.2) (layer "F.Cu") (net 13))
 (segment (start 132.368 101.7357) (end 133.2317 102.5994) (width 0.2) (layer "F.Cu") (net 13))
 (segment (start 133.2317 102.5994) (end 133.2317 117.826) (width 0.2) (layer "F.Cu") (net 13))
 (segment (start 132.08 100.584) (end 132.08 101.7357) (width 0.2) (layer "F.Cu") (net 13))
 (segment (start 132.08 101.7357) (end 132.368 101.7357) (width 0.2) (layer "F.Cu") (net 13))
 (segment (start 166.6422 138.0241) (end 167.416 138.7979) (width 0.2) (layer "B.Cu") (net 2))
 (segment (start 168.2027 140.3568) (end 181.878 140.3568) (width 0.2) (layer "B.Cu") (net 2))
 (segment (start 154.94 123.8913) (end 153.7217 125.1096) (width 0.2) (layer "B.Cu") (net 2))
 (segment (start 164.876 136.2639) (end 164.876 137.0331) (width 0.2) (layer "B.Cu") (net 2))
 (segment (start 154.94 103.124) (end 154.94 123.8913) (width 0.2) (layer "B.Cu") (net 2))
 (segment (start 142.016 136.2426) (end 153.149 125.1096) (width 0.2) (layer "B.Cu") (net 2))
 (segment (start 181.878 140.3568) (end 182.7743 139.4605) (width 0.2) (layer "B.Cu") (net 2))
 (segment (start 124.1177 139.192) (end 124.1177 138.9235) (width 0.2) (layer "B.Cu") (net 2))
 (segment (start 142.016 137.0973) (end 142.016 136.2426) (width 0.2) (layer "B.Cu") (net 2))
 (segment (start 153.7217 125.1096) (end 164.876 136.2639) (width 0.2) (layer "B.Cu") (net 2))
 (segment (start 124.1177 138.9235) (end 125.1192 137.922) (width 0.2) (layer "B.Cu") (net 2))
 (segment (start 167.416 138.7979) (end 167.416 139.5701) (width 0.2) (layer "B.Cu") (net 2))
 (segment (start 164.876 137.0331) (end 165.867 138.0241) (width 0.2) (layer "B.Cu") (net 2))
 (segment (start 122.966 139.192) (end 124.1177 139.192) (width 0.2) (layer "B.Cu") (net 2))
 (segment (start 182.7743 139.4605) (end 182.7743 139.192) (width 0.2) (layer "B.Cu") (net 2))
 (segment (start 183.926 139.192) (end 182.7743 139.192) (width 0.2) (layer "B.Cu") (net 2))
 (segment (start 141.1913 137.922) (end 142.016 137.0973) (width 0.2) (layer "B.Cu") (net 2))
 (segment (start 153.149 125.1096) (end 153.7217 125.1096) (width 0.2) (layer "B.Cu") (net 2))
 (segment (start 167.416 139.5701) (end 168.2027 140.3568) (width 0.2) (layer "B.Cu") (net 2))
 (segment (start 125.1192 137.922) (end 141.1913 137.922) (width 0.2) (layer "B.Cu") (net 2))
 (segment (start 165.867 138.0241) (end 166.6422 138.0241) (width 0.2) (layer "B.Cu") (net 2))
 (segment (start 134.62 116.6743) (end 153.446 135.5003) (width 0.2) (layer "F.Cu") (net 14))
 (segment (start 153.446 136.652) (end 153.446 135.5003) (width 0.2) (layer "F.Cu") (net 14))
 (segment (start 134.62 103.124) (end 134.62 116.6743) (width 0.2) (layer "F.Cu") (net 14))
 (segment (start 139.7 118.7663) (end 122.966 135.5003) (width 0.2) (layer "B.Cu") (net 1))
 (segment (start 139.7 103.124) (end 139.7 118.7663) (width 0.2) (layer "B.Cu") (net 1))
 (segment (start 122.966 136.652) (end 122.966 135.5003) (width 0.2) (layer "B.Cu") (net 1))
 (segment (start 142.24 103.124) (end 142.24 121.3063) (width 0.2) (layer "B.Cu") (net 4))
 (segment (start 128.046 136.652) (end 128.046 135.5003) (width 0.2) (layer "B.Cu") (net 4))
 (segment (start 142.24 121.3063) (end 128.046 135.5003) (width 0.2) (layer "B.Cu") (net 4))
 (segment (start 160.02 101.7357) (end 160.308 101.7357) (width 0.2) (layer "B.Cu") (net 21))
 (segment (start 161.1717 125.446) (end 171.226 135.5003) (width 0.2) (layer "B.Cu") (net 21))
 (segment (start 171.226 136.652) (end 171.226 135.5003) (width 0.2) (layer "B.Cu") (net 21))
 (segment (start 160.02 100.584) (end 160.02 101.7357) (width 0.2) (layer "B.Cu") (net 21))
 (segment (start 160.308 101.7357) (end 161.1717 102.5994) (width 0.2) (layer "B.Cu") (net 21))
 (segment (start 161.1717 102.5994) (end 161.1717 125.446) (width 0.2) (layer "B.Cu") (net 21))
 (segment (start 149.86 103.124) (end 151.0117 103.124) (width 0.2) (layer "F.Cu") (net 26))
 (segment (start 180.7273 129.7795) (end 180.7273 130.048) (width 0.2) (layer "F.Cu") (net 26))
 (segment (start 181.879 130.048) (end 180.7273 130.048) (width 0.2) (layer "F.Cu") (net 26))
 (segment (start 155.2235 104.2757) (end 180.7273 129.7795) (width 0.2) (layer "F.Cu") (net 26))
 (segment (start 151.0117 103.124) (end 151.0117 103.412) (width 0.2) (layer "F.Cu") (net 26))
 (segment (start 151.8754 104.2757) (end 155.2235 104.2757) (width 0.2) (layer "F.Cu") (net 26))
 (segment (start 151.0117 103.412) (end 151.8754 104.2757) (width 0.2) (layer "F.Cu") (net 26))
 (segment (start 145.826 136.652) (end 145.826 135.5003) (width 0.2) (layer "F.Cu") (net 11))
 (segment (start 130.3318 101.7357) (end 130.6917 102.0956) (width 0.2) (layer "F.Cu") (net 11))
 (segment (start 129.54 101.7357) (end 130.3318 101.7357) (width 0.2) (layer "F.Cu") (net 11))
 (segment (start 129.54 100.584) (end 129.54 101.7357) (width 0.2) (layer "F.Cu") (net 11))
 (segment (start 130.6917 102.0956) (end 130.6917 120.366) (width 0.2) (layer "F.Cu") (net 11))
 (segment (start 130.6917 120.366) (end 145.826 135.5003) (width 0.2) (layer "F.Cu") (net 11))
 (segment (start 179.339 132.4673) (end 176.306 135.5003) (width 0.2) (layer "B.Cu") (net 23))
 (segment (start 179.339 130.048) (end 179.339 132.4673) (width 0.2) (layer "B.Cu") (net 23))
 (segment (start 176.306 136.652) (end 176.306 135.5003) (width 0.2) (layer "B.Cu") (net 23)))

